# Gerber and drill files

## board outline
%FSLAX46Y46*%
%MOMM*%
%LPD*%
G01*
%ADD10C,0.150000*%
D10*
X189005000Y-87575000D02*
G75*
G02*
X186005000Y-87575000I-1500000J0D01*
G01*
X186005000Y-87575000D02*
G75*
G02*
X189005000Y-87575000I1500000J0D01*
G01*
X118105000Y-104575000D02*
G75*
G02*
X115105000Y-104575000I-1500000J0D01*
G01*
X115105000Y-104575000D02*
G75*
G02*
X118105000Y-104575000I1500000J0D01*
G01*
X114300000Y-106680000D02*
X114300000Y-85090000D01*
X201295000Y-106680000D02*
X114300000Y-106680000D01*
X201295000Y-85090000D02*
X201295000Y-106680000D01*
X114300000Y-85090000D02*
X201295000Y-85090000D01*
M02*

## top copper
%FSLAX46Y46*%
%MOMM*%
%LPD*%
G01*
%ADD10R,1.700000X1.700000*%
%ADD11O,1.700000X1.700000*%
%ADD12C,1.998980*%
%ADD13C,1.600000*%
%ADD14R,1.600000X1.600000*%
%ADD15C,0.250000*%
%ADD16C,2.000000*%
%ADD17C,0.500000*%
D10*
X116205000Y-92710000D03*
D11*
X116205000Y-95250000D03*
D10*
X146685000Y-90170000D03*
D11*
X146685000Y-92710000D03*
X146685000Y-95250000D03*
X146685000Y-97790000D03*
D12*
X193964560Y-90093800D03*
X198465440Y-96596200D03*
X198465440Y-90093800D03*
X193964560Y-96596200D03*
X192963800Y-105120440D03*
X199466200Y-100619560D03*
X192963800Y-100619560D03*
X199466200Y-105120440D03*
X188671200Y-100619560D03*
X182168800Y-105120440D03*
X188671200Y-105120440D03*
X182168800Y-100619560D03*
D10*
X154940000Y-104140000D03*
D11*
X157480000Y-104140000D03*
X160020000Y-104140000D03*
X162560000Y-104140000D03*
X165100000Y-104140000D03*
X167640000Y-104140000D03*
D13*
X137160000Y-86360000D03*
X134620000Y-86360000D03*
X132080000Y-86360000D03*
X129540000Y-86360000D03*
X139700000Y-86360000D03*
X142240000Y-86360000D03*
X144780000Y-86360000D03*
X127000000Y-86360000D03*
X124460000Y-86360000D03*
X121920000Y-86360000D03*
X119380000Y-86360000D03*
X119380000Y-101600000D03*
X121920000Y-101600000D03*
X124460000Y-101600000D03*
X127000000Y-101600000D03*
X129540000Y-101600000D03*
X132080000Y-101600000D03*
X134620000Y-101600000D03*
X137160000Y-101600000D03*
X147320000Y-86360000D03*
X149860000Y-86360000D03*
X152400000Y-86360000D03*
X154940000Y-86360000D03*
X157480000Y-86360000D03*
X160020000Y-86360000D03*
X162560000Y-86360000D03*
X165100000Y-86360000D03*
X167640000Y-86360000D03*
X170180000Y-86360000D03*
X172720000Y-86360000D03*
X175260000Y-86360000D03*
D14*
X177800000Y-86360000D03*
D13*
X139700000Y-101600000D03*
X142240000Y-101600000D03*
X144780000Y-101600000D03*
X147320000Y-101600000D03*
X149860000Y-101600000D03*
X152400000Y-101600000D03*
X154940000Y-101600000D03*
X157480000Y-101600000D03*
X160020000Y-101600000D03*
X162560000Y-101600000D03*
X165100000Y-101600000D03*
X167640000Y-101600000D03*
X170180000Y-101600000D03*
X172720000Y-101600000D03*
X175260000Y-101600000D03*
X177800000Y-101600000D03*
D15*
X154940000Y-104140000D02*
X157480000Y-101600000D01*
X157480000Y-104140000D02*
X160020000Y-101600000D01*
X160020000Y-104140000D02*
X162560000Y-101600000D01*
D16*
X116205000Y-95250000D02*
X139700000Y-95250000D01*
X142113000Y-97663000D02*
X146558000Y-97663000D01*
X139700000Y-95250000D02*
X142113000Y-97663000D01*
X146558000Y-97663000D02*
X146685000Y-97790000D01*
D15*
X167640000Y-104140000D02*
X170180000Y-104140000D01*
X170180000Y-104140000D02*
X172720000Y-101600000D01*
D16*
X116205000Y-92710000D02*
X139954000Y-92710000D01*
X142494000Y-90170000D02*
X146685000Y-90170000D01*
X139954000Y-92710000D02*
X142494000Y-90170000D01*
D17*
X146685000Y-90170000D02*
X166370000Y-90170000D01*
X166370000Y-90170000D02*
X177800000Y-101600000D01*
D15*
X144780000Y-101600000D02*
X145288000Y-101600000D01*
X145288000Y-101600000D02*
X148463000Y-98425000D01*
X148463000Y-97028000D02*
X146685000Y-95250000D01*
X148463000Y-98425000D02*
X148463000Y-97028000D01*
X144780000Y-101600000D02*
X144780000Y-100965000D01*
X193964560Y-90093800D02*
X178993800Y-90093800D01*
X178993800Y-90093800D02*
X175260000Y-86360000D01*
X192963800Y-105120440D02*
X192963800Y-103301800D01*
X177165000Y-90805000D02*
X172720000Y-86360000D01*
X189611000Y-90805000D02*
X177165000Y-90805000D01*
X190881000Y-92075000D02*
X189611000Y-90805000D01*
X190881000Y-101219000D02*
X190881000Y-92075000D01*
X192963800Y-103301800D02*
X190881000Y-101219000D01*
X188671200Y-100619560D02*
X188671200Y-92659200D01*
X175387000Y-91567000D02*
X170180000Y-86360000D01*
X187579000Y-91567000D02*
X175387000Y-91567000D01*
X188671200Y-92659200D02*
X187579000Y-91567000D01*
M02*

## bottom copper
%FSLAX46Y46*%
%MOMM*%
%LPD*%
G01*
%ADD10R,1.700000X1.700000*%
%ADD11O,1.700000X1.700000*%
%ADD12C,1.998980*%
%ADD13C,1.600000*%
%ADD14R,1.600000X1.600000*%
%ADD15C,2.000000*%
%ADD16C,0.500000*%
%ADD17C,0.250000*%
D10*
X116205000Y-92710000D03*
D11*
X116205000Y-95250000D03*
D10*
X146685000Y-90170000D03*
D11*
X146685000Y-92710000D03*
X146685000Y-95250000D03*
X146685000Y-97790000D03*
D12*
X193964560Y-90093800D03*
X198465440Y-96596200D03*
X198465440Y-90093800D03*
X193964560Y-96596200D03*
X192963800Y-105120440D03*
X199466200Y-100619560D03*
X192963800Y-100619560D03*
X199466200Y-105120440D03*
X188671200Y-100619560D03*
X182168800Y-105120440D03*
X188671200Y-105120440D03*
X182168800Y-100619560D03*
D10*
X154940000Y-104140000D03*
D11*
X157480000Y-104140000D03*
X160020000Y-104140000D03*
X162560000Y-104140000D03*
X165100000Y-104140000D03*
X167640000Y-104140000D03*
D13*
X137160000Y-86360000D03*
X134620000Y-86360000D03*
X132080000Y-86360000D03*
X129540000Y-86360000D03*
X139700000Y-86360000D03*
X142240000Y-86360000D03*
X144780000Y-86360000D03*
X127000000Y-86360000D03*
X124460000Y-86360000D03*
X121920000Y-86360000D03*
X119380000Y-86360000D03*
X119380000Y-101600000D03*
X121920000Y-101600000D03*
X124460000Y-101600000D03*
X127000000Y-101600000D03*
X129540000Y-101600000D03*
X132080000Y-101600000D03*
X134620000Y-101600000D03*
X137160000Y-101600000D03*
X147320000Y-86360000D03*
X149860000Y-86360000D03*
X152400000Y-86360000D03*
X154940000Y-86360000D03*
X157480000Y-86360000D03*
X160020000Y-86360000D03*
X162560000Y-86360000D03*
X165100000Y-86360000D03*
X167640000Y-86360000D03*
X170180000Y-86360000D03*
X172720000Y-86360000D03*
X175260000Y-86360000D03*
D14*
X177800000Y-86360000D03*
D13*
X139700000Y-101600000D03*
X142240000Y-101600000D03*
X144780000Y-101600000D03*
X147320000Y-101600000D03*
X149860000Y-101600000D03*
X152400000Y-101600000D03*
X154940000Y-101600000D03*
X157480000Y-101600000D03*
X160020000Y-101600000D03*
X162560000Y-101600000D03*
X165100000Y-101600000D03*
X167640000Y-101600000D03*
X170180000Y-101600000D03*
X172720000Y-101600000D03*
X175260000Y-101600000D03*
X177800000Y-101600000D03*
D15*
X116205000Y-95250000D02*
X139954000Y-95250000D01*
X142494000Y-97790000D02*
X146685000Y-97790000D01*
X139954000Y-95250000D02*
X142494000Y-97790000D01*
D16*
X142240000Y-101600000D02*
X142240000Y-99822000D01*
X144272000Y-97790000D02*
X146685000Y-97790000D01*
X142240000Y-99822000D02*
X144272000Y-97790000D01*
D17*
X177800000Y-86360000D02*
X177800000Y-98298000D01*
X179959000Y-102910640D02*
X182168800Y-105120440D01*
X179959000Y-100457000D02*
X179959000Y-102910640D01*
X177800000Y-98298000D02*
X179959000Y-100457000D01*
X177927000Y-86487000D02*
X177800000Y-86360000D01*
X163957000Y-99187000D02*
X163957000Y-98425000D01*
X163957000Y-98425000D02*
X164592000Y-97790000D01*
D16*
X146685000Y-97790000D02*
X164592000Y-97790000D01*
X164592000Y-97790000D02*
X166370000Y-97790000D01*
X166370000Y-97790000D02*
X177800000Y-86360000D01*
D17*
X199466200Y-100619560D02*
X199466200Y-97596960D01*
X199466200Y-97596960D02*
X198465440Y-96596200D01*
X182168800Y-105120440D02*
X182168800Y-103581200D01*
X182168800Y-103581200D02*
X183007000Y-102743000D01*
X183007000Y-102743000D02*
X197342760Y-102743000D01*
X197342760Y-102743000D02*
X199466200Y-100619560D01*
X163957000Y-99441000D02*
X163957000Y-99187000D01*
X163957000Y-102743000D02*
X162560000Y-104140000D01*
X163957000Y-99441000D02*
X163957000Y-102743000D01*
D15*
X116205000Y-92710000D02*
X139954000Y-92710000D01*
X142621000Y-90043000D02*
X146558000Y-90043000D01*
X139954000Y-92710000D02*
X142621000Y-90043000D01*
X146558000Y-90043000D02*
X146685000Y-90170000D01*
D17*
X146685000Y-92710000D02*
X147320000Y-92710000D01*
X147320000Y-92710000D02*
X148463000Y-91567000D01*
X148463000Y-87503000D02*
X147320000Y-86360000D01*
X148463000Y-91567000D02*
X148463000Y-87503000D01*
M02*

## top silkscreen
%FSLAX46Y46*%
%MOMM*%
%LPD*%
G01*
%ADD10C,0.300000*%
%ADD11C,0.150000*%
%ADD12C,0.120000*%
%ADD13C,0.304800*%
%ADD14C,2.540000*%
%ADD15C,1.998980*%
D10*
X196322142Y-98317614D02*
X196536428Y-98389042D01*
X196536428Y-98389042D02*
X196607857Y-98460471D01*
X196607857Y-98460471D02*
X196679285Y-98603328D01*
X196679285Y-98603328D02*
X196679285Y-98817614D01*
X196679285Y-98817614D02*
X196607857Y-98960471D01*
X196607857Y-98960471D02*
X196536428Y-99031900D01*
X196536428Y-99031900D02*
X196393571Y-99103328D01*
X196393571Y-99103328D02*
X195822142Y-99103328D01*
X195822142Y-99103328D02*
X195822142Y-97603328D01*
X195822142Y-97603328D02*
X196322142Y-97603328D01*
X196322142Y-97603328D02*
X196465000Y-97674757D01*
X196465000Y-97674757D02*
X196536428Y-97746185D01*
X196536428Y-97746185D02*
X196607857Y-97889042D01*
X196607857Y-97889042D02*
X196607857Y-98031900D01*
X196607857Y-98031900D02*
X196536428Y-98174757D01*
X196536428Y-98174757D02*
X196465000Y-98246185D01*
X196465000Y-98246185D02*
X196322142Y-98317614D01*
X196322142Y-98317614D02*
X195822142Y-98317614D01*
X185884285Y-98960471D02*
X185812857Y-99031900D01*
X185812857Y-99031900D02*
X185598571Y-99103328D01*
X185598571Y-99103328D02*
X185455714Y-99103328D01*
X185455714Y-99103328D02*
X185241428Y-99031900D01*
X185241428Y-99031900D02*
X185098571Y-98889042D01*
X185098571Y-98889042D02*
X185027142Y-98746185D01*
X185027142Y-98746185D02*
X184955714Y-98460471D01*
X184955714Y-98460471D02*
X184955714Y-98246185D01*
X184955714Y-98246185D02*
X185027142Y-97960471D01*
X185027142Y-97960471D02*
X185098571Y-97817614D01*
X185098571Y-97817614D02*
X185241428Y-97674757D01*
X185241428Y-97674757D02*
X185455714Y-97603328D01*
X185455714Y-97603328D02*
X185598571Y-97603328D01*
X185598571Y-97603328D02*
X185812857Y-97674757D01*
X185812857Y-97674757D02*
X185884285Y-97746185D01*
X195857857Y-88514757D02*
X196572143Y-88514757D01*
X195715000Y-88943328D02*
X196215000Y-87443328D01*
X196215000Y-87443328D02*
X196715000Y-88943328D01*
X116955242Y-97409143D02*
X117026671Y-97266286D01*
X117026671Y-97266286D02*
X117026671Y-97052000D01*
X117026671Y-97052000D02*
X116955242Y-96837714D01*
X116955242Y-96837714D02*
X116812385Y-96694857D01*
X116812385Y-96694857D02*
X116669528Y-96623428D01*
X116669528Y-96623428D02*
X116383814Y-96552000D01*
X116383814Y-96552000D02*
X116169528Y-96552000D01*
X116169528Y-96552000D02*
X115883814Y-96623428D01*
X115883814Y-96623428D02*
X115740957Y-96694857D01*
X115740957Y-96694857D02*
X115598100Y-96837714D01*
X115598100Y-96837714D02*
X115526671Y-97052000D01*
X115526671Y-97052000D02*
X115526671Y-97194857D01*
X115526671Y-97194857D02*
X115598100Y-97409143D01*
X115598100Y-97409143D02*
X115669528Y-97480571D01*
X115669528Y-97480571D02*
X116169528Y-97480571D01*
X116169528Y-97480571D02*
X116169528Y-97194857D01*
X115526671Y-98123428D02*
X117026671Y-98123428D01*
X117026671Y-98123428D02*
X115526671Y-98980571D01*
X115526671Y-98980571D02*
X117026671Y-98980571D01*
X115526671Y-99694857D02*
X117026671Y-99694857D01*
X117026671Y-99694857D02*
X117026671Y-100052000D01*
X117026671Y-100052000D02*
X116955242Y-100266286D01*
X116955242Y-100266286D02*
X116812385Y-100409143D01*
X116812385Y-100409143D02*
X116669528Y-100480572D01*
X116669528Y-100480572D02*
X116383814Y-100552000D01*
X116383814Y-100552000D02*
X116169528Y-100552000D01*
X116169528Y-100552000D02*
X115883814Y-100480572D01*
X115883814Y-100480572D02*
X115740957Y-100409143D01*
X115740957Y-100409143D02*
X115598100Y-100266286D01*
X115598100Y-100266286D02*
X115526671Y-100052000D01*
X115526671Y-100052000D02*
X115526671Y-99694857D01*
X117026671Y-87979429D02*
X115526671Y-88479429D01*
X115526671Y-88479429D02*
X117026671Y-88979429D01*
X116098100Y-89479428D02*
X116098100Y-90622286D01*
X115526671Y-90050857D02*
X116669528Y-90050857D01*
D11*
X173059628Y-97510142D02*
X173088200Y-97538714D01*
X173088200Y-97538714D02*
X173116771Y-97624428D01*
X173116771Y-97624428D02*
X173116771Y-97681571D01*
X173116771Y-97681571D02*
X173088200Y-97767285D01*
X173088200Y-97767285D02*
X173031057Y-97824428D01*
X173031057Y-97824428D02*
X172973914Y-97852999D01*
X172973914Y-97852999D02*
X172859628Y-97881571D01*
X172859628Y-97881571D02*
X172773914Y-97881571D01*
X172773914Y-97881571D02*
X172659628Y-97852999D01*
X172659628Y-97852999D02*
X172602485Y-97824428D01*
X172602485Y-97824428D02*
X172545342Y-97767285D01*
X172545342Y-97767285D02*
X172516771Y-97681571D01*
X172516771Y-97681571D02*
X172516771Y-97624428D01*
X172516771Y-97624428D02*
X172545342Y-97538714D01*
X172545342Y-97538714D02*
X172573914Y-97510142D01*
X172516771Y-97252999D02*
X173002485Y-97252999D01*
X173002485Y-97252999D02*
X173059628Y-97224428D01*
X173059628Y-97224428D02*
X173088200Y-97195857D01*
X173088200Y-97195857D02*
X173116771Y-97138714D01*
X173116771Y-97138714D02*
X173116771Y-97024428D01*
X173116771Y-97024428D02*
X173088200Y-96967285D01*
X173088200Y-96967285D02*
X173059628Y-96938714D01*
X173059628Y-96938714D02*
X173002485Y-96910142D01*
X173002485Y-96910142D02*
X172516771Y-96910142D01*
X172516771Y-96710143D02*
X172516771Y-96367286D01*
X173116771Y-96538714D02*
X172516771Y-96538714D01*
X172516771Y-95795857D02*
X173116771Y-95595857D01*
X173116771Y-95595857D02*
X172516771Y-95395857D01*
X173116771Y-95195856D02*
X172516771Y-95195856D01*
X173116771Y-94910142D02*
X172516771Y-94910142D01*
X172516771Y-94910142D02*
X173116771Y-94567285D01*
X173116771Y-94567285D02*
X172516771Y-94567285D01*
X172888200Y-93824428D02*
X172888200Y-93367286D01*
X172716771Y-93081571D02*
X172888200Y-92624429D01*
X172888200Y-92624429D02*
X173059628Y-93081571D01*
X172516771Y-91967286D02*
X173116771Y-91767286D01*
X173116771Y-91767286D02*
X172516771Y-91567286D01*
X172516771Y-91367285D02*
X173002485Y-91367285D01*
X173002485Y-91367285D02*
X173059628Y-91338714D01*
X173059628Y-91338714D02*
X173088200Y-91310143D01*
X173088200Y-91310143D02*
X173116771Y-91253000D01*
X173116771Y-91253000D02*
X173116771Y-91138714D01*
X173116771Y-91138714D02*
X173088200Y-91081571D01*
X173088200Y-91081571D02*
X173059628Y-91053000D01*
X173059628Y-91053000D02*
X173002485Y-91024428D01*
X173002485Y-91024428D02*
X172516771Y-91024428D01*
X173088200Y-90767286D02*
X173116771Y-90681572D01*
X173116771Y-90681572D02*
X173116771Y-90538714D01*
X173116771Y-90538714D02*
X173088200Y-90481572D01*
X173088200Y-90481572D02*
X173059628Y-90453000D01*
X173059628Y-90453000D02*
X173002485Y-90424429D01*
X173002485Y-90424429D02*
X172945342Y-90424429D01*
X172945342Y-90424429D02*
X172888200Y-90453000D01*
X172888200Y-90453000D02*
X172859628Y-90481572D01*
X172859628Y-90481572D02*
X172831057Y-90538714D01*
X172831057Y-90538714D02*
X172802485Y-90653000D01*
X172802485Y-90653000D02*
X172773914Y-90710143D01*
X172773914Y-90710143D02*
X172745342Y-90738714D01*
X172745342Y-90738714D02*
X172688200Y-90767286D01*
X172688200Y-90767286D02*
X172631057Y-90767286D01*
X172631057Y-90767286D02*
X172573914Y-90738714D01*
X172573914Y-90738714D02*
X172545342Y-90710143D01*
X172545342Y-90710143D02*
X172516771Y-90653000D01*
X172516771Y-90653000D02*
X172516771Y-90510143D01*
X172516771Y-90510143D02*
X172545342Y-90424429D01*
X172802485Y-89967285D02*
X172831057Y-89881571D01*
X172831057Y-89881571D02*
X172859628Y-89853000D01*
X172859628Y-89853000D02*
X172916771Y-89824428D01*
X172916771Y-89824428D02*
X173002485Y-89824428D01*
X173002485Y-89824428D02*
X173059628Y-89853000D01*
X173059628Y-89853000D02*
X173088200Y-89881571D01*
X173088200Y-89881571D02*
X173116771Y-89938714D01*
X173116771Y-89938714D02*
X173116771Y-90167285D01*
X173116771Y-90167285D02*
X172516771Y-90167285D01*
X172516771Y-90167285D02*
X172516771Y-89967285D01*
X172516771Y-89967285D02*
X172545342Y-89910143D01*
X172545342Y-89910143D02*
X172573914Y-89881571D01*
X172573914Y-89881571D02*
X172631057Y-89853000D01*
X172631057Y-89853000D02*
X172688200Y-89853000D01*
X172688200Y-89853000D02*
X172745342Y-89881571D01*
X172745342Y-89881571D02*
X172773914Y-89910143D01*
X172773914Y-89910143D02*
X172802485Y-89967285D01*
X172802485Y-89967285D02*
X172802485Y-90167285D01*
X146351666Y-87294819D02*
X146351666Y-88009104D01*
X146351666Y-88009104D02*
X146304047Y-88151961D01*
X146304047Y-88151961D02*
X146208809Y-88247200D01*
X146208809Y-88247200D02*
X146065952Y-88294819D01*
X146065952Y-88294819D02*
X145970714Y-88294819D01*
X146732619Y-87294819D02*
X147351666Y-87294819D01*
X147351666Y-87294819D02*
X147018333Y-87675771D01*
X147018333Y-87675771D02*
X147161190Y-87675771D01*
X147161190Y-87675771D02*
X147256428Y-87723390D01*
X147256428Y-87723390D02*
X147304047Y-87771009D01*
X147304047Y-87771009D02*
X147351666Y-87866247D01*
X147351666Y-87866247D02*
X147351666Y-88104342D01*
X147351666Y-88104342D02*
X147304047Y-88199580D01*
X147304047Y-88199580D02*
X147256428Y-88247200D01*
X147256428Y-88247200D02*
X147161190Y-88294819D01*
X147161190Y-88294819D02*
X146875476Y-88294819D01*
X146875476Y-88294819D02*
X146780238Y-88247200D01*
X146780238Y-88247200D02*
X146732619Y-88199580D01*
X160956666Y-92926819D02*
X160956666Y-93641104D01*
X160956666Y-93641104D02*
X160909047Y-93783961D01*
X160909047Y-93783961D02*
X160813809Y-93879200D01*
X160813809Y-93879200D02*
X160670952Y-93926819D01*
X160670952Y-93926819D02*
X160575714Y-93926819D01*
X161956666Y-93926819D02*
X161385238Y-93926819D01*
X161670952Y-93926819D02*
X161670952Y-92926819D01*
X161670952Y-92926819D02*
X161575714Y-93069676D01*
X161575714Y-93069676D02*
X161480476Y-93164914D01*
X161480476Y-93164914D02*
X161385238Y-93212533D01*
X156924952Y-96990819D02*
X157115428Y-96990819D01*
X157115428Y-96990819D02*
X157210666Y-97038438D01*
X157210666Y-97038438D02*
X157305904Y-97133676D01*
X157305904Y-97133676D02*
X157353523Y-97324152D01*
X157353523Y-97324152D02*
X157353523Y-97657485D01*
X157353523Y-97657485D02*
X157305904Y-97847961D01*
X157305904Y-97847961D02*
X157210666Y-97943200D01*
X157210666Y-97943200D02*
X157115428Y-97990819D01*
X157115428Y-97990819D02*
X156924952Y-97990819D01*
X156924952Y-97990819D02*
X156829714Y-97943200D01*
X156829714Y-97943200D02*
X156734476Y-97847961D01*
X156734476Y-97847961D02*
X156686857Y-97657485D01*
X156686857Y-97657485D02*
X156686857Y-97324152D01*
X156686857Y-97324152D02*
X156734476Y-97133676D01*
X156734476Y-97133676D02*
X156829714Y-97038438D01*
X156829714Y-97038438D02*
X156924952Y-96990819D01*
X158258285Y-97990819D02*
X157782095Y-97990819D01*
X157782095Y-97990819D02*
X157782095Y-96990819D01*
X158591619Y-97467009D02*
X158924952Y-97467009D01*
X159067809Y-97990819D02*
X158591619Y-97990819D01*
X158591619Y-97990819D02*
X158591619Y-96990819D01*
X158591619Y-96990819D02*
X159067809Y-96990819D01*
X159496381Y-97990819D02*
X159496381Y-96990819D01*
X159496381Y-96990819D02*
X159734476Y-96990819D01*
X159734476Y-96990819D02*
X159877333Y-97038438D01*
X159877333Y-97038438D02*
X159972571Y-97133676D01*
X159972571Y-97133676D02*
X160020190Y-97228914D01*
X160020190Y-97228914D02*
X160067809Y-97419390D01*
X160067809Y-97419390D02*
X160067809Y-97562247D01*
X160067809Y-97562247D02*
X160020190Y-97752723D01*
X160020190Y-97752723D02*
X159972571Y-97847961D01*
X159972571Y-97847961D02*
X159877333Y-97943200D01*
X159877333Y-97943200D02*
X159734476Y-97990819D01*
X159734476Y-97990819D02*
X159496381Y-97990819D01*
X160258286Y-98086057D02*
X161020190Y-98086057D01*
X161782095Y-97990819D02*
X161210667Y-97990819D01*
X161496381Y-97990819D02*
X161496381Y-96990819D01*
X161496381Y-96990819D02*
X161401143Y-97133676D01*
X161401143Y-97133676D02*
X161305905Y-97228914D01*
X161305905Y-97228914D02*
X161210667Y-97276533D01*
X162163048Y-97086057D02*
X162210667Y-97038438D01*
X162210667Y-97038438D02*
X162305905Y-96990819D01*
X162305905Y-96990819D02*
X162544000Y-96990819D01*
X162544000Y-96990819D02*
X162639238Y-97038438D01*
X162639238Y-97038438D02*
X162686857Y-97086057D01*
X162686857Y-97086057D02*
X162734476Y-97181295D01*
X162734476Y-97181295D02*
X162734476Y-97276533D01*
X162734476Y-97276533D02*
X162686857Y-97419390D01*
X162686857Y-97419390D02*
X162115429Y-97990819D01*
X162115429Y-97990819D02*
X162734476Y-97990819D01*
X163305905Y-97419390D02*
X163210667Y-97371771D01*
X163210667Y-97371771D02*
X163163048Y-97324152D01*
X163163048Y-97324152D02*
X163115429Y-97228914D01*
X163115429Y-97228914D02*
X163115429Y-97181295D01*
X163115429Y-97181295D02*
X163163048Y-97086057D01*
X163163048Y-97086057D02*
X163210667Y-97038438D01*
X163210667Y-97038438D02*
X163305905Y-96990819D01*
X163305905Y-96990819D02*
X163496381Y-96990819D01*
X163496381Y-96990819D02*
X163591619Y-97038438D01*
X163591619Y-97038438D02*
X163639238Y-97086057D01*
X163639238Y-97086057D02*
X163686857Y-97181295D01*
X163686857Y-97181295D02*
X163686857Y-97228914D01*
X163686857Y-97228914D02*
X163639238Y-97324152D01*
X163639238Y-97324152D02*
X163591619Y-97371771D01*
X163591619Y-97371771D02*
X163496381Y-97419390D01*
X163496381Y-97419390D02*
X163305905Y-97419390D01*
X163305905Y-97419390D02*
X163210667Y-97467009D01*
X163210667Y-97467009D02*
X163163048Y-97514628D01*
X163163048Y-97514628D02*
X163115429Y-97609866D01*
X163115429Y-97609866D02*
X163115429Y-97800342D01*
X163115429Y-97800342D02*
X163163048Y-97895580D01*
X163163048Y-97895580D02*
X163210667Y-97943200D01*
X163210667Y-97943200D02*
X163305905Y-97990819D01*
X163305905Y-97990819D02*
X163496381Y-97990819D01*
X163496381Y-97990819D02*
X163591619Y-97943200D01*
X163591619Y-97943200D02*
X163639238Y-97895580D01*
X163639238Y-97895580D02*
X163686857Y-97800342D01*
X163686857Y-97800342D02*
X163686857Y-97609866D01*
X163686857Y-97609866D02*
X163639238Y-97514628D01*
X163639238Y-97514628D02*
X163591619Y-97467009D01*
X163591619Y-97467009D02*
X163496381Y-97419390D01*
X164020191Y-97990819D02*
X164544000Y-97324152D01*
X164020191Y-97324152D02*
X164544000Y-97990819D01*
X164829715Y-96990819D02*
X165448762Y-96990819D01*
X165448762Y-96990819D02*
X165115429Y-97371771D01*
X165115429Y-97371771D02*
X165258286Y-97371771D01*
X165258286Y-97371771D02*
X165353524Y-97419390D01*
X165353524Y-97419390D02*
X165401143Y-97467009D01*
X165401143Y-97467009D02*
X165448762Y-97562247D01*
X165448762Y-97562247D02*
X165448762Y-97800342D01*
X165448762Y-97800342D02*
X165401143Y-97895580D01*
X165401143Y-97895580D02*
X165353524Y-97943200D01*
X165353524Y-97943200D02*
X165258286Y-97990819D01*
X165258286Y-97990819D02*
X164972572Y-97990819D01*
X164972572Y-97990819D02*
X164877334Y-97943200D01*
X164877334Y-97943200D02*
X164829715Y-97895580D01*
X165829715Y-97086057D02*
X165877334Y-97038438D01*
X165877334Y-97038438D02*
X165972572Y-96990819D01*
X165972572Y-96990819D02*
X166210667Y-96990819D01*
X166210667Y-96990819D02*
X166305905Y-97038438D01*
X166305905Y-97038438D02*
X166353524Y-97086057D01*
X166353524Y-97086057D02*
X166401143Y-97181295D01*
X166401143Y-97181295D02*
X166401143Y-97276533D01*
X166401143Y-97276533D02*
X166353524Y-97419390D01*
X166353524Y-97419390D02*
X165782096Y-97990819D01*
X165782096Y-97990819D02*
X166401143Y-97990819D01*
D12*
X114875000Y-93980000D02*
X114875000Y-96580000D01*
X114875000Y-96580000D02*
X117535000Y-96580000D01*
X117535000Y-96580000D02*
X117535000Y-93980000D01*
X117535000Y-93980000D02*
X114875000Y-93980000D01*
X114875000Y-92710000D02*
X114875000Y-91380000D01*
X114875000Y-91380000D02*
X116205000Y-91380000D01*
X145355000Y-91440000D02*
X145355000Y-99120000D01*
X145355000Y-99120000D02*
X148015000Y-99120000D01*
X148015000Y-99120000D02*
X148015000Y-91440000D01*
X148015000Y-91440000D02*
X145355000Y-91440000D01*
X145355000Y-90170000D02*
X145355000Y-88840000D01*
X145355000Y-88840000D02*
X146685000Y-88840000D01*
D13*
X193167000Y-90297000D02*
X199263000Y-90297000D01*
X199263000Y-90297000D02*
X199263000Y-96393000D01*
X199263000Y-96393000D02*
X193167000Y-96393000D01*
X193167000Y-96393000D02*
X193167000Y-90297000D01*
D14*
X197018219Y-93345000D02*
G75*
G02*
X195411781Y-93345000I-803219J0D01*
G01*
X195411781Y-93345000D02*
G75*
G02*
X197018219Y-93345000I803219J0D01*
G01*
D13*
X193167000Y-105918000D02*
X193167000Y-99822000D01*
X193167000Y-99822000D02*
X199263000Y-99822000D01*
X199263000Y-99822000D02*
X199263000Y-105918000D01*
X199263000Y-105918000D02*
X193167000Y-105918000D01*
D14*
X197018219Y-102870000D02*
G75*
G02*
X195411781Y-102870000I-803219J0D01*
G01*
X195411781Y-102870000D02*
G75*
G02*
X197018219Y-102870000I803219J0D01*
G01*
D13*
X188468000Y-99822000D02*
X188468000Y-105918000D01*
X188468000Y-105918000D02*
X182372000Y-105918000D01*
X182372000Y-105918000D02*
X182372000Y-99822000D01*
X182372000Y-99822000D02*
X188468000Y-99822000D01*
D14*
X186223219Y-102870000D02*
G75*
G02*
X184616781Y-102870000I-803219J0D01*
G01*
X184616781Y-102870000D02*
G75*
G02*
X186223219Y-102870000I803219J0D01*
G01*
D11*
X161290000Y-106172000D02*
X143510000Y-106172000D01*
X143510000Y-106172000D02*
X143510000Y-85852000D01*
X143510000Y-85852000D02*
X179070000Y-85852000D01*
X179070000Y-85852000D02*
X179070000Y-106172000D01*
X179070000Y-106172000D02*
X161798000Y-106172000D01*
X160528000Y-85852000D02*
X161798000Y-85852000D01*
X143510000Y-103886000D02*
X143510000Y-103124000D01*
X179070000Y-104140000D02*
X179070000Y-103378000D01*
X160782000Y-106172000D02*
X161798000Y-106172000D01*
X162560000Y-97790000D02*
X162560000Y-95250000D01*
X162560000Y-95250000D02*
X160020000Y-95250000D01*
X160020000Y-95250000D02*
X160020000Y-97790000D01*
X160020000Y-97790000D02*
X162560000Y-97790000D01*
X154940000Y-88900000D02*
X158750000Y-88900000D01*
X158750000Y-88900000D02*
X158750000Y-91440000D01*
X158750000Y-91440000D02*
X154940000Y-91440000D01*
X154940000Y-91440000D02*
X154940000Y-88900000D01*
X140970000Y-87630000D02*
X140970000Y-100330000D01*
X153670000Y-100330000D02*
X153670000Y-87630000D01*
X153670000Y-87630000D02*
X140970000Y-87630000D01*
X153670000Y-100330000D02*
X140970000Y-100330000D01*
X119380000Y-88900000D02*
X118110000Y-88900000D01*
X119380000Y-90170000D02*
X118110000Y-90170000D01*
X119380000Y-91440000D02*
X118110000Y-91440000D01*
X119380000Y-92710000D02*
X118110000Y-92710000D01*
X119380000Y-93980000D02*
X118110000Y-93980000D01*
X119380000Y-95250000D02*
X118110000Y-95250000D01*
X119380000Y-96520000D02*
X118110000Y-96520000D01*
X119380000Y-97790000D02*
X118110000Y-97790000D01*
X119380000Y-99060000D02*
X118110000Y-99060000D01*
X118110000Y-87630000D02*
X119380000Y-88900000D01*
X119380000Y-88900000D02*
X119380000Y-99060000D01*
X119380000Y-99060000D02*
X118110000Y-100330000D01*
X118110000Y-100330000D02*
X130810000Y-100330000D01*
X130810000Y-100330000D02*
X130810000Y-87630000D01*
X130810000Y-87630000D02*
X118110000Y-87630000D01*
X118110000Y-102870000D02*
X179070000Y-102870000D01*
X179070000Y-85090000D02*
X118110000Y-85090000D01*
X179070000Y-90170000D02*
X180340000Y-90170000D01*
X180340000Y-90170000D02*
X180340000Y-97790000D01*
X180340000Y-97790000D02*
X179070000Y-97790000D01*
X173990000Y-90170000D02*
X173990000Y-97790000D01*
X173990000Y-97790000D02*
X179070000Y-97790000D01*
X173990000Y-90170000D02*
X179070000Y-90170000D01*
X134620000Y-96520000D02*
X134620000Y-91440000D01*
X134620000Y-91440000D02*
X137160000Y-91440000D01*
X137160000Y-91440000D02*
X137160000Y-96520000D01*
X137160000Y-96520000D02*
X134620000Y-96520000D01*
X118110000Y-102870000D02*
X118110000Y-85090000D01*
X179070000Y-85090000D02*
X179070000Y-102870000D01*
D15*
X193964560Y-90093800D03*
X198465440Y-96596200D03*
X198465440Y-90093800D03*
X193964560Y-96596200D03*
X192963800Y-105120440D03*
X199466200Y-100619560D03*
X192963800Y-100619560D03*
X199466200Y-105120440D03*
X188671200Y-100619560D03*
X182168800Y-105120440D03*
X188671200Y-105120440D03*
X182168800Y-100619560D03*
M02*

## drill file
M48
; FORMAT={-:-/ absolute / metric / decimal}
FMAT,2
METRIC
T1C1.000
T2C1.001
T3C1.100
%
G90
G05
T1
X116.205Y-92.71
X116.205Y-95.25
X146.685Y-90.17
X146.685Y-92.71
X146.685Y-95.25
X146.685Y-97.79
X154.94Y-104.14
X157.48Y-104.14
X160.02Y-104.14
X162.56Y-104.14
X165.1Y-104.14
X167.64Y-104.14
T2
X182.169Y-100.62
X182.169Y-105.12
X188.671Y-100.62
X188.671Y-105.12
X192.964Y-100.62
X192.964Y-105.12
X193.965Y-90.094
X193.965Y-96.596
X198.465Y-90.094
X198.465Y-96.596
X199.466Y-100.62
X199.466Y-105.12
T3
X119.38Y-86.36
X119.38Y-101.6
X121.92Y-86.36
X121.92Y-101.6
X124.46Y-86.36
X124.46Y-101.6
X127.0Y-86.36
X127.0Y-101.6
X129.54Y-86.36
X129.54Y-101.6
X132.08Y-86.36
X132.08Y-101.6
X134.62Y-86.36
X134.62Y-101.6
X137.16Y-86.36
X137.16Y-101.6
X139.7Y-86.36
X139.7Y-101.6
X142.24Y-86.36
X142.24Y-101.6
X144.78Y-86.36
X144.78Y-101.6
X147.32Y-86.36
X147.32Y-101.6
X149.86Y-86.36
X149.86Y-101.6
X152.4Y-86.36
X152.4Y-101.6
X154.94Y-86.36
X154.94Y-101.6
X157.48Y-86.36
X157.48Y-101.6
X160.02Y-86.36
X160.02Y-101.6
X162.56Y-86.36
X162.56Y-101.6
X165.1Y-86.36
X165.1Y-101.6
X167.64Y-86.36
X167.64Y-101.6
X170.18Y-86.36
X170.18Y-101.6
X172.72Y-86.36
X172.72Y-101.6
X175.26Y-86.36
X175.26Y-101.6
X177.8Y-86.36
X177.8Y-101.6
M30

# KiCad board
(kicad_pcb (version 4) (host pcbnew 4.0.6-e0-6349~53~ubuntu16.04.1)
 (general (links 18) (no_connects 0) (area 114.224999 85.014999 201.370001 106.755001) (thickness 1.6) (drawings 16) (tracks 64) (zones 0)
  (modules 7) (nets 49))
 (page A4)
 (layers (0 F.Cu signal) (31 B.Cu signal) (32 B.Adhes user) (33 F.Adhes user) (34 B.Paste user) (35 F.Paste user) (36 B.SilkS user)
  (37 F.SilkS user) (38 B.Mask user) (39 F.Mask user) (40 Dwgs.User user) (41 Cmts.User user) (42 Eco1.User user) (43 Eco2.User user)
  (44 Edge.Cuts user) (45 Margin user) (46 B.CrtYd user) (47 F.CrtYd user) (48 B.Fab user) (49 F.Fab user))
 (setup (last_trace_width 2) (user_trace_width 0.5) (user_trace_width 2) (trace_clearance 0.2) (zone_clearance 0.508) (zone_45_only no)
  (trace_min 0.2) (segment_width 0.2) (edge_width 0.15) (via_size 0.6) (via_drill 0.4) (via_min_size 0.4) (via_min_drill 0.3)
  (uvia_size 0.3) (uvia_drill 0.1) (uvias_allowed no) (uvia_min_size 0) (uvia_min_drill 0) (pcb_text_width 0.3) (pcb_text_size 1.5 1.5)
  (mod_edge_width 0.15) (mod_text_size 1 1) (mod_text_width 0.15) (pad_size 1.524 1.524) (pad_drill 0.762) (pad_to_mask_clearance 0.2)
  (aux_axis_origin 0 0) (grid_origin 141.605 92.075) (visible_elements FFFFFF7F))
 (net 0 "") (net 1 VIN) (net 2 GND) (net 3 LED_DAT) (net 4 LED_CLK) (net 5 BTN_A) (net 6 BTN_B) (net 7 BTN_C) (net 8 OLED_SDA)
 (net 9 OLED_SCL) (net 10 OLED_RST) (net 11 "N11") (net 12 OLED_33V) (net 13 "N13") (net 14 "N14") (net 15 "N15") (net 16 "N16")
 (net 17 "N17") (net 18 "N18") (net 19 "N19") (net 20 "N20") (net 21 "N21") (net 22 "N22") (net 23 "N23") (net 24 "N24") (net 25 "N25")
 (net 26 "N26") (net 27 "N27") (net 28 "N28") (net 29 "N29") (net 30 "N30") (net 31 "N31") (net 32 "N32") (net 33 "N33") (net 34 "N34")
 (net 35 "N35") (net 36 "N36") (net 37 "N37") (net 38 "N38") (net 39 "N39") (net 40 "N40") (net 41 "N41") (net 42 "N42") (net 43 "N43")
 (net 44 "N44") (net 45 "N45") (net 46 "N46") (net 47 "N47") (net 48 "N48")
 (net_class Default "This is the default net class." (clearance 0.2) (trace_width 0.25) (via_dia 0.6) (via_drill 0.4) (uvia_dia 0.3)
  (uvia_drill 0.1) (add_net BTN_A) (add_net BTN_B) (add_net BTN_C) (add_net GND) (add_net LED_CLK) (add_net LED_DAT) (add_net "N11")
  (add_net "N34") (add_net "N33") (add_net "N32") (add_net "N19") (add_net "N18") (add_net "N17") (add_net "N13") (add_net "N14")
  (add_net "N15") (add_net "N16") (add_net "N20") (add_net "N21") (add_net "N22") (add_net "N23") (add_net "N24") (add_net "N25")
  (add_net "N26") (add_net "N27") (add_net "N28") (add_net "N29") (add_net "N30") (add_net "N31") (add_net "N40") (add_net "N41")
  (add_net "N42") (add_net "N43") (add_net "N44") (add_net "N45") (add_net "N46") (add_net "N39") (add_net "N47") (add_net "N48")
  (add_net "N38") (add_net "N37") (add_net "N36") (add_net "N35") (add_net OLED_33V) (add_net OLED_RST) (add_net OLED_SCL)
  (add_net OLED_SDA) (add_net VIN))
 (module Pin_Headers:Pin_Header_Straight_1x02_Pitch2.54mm (layer F.Cu) (at 116.205 92.71)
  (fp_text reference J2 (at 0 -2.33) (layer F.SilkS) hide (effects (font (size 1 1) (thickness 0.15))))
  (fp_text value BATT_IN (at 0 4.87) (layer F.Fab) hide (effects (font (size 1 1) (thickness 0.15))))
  (fp_line (start -1.33 1.27) (end -1.33 3.87) (layer F.SilkS) (width 0.12))
  (fp_line (start -1.33 3.87) (end 1.33 3.87) (layer F.SilkS) (width 0.12))
  (fp_line (start 1.33 3.87) (end 1.33 1.27) (layer F.SilkS) (width 0.12))
  (fp_line (start 1.33 1.27) (end -1.33 1.27) (layer F.SilkS) (width 0.12))
  (fp_line (start -1.33 0) (end -1.33 -1.33) (layer F.SilkS) (width 0.12))
  (fp_line (start -1.33 -1.33) (end 0 -1.33) (layer F.SilkS) (width 0.12))
  (pad 1 thru_hole rect (at 0 0) (size 1.7 1.7) (drill 1) (layers *.Cu *.Mask) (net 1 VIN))
  (pad 2 thru_hole oval (at 0 2.54) (size 1.7 1.7) (drill 1) (layers *.Cu *.Mask) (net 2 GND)))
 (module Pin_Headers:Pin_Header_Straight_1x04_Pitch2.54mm (layer F.Cu) (at 146.685 90.17)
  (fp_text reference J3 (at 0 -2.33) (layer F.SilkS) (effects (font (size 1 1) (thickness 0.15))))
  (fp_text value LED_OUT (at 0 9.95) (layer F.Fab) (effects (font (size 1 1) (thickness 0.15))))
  (fp_line (start -1.33 1.27) (end -1.33 8.95) (layer F.SilkS) (width 0.12))
  (fp_line (start -1.33 8.95) (end 1.33 8.95) (layer F.SilkS) (width 0.12))
  (fp_line (start 1.33 8.95) (end 1.33 1.27) (layer F.SilkS) (width 0.12))
  (fp_line (start 1.33 1.27) (end -1.33 1.27) (layer F.SilkS) (width 0.12))
  (fp_line (start -1.33 0) (end -1.33 -1.33) (layer F.SilkS) (width 0.12))
  (fp_line (start -1.33 -1.33) (end 0 -1.33) (layer F.SilkS) (width 0.12))
  (pad 1 thru_hole rect (at 0 0) (size 1.7 1.7) (drill 1) (layers *.Cu *.Mask) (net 1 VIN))
  (pad 2 thru_hole oval (at 0 2.54) (size 1.7 1.7) (drill 1) (layers *.Cu *.Mask) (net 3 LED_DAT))
  (pad 3 thru_hole oval (at 0 5.08) (size 1.7 1.7) (drill 1) (layers *.Cu *.Mask) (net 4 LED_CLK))
  (pad 4 thru_hole oval (at 0 7.62) (size 1.7 1.7) (drill 1) (layers *.Cu *.Mask) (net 2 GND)))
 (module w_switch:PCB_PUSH (layer F.Cu) (at 196.215 93.345)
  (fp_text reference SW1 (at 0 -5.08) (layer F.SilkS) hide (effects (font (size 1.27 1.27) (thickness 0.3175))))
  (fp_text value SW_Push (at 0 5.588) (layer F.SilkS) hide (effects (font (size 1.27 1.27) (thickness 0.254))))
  (fp_line (start -3.048 -3.048) (end 3.048 -3.048) (layer F.SilkS) (width 0.3048))
  (fp_line (start 3.048 -3.048) (end 3.048 3.048) (layer F.SilkS) (width 0.3048))
  (fp_line (start 3.048 3.048) (end -3.048 3.048) (layer F.SilkS) (width 0.3048))
  (fp_line (start -3.048 3.048) (end -3.048 -3.048) (layer F.SilkS) (width 0.3048))
  (fp_circle (center 0 0) (end -0.762 0.254) (layer F.SilkS) (width 2.54))
  (pad 1 thru_hole circle (at -2.25044 -3.2512) (size 1.99898 1.99898) (drill 1.00076) (layers *.Cu *.Mask F.SilkS) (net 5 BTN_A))
  (pad 2 thru_hole circle (at 2.25044 3.2512) (size 1.99898 1.99898) (drill 1.00076) (layers *.Cu *.Mask F.SilkS) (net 2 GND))
  (pad 4 thru_hole circle (at 2.25044 -3.2512) (size 1.99898 1.99898) (drill 1.00076) (layers *.Cu *.Mask F.SilkS))
  (pad 3 thru_hole circle (at -2.25044 3.2512) (size 1.99898 1.99898) (drill 1.00076) (layers *.Cu *.Mask F.SilkS)))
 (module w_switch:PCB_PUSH (layer F.Cu) (at 196.215 102.87 90)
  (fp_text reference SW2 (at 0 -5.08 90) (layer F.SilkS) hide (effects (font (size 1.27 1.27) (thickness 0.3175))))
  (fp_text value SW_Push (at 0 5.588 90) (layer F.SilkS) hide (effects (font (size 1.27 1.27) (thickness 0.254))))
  (fp_line (start -3.048 -3.048) (end 3.048 -3.048) (layer F.SilkS) (width 0.3048))
  (fp_line (start 3.048 -3.048) (end 3.048 3.048) (layer F.SilkS) (width 0.3048))
  (fp_line (start 3.048 3.048) (end -3.048 3.048) (layer F.SilkS) (width 0.3048))
  (fp_line (start -3.048 3.048) (end -3.048 -3.048) (layer F.SilkS) (width 0.3048))
  (fp_circle (center 0 0) (end -0.762 0.254) (layer F.SilkS) (width 2.54))
  (pad 1 thru_hole circle (at -2.25044 -3.2512 90) (size 1.99898 1.99898) (drill 1.00076) (layers *.Cu *.Mask F.SilkS) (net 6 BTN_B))
  (pad 2 thru_hole circle (at 2.25044 3.2512 90) (size 1.99898 1.99898) (drill 1.00076) (layers *.Cu *.Mask F.SilkS) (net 2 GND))
  (pad 4 thru_hole circle (at 2.25044 -3.2512 90) (size 1.99898 1.99898) (drill 1.00076) (layers *.Cu *.Mask F.SilkS))
  (pad 3 thru_hole circle (at -2.25044 3.2512 90) (size 1.99898 1.99898) (drill 1.00076) (layers *.Cu *.Mask F.SilkS)))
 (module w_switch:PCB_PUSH (layer F.Cu) (at 185.42 102.87 270)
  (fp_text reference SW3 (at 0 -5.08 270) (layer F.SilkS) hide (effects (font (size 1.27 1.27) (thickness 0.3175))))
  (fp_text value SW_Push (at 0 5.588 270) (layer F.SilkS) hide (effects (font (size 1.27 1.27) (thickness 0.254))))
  (fp_line (start -3.048 -3.048) (end 3.048 -3.048) (layer F.SilkS) (width 0.3048))
  (fp_line (start 3.048 -3.048) (end 3.048 3.048) (layer F.SilkS) (width 0.3048))
  (fp_line (start 3.048 3.048) (end -3.048 3.048) (layer F.SilkS) (width 0.3048))
  (fp_line (start -3.048 3.048) (end -3.048 -3.048) (layer F.SilkS) (width 0.3048))
  (fp_circle (center 0 0) (end -0.762 0.254) (layer F.SilkS) (width 2.54))
  (pad 1 thru_hole circle (at -2.25044 -3.2512 270) (size 1.99898 1.99898) (drill 1.00076) (layers *.Cu *.Mask F.SilkS) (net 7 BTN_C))
  (pad 2 thru_hole circle (at 2.25044 3.2512 270) (size 1.99898 1.99898) (drill 1.00076) (layers *.Cu *.Mask F.SilkS) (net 2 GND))
  (pad 4 thru_hole circle (at 2.25044 -3.2512 270) (size 1.99898 1.99898) (drill 1.00076) (layers *.Cu *.Mask F.SilkS))
  (pad 3 thru_hole circle (at -2.25044 3.2512 270) (size 1.99898 1.99898) (drill 1.00076) (layers *.Cu *.Mask F.SilkS)))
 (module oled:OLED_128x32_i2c (layer F.Cu) (at 161.29 104.14)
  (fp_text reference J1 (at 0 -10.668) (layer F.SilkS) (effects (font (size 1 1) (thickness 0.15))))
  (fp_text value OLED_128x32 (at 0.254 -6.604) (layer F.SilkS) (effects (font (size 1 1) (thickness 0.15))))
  (fp_line (start 0 2.032) (end -17.78 2.032) (layer F.SilkS) (width 0.15))
  (fp_line (start -17.78 2.032) (end -17.78 -18.288) (layer F.SilkS) (width 0.15))
  (fp_line (start -17.78 -18.288) (end 17.78 -18.288) (layer F.SilkS) (width 0.15))
  (fp_line (start 17.78 -18.288) (end 17.78 2.032) (layer F.SilkS) (width 0.15))
  (fp_line (start 17.78 2.032) (end 0.508 2.032) (layer F.SilkS) (width 0.15))
  (fp_line (start -0.762 -18.288) (end 0.508 -18.288) (layer F.SilkS) (width 0.15))
  (fp_line (start -17.78 -0.254) (end -17.78 -1.016) (layer F.SilkS) (width 0.15))
  (fp_line (start 17.78 0) (end 17.78 -0.762) (layer F.SilkS) (width 0.15))
  (fp_line (start -0.508 2.032) (end 0.508 2.032) (layer F.SilkS) (width 0.15))
  (pad 1 thru_hole rect (at -6.35 0) (size 1.7 1.7) (drill 1) (layers *.Cu *.Mask) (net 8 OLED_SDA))
  (pad 2 thru_hole oval (at -3.81 0) (size 1.7 1.7) (drill 1) (layers *.Cu *.Mask) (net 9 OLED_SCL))
  (pad 3 thru_hole oval (at -1.27 0) (size 1.7 1.7) (drill 1) (layers *.Cu *.Mask) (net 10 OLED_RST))
  (pad 4 thru_hole oval (at 1.27 0) (size 1.7 1.7) (drill 1) (layers *.Cu *.Mask) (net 2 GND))
  (pad 5 thru_hole oval (at 3.81 0) (size 1.7 1.7) (drill 1) (layers *.Cu *.Mask) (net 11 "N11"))
  (pad 6 thru_hole oval (at 6.35 0) (size 1.7 1.7) (drill 1) (layers *.Cu *.Mask) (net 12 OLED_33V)))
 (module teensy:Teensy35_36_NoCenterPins (layer F.Cu) (at 148.59 93.98 180)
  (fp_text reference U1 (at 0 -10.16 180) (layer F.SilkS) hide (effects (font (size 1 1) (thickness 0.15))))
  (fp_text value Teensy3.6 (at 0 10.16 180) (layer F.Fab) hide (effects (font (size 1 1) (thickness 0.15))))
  (fp_line (start -13.97 -3.81) (end -13.97 -1.27) (layer F.SilkS) (width 0.15))
  (fp_line (start -13.97 -1.27) (end -11.43 -1.27) (layer F.SilkS) (width 0.15))
  (fp_line (start -11.43 -1.27) (end -11.43 -3.81) (layer F.SilkS) (width 0.15))
  (fp_line (start -11.43 -3.81) (end -13.97 -3.81) (layer F.SilkS) (width 0.15))
  (fp_line (start -6.35 5.08) (end -10.16 5.08) (layer F.SilkS) (width 0.15))
  (fp_line (start -10.16 5.08) (end -10.16 2.54) (layer F.SilkS) (width 0.15))
  (fp_line (start -10.16 2.54) (end -6.35 2.54) (layer F.SilkS) (width 0.15))
  (fp_line (start -6.35 2.54) (end -6.35 5.08) (layer F.SilkS) (width 0.15))
  (fp_line (start 7.62 6.35) (end 7.62 -6.35) (layer F.SilkS) (width 0.15))
  (fp_line (start -5.08 -6.35) (end -5.08 6.35) (layer F.SilkS) (width 0.15))
  (fp_line (start -5.08 6.35) (end 7.62 6.35) (layer F.SilkS) (width 0.15))
  (fp_line (start -5.08 -6.35) (end 7.62 -6.35) (layer F.SilkS) (width 0.15))
  (fp_line (start 29.21 5.08) (end 30.48 5.08) (layer F.SilkS) (width 0.15))
  (fp_line (start 29.21 3.81) (end 30.48 3.81) (layer F.SilkS) (width 0.15))
  (fp_line (start 29.21 2.54) (end 30.48 2.54) (layer F.SilkS) (width 0.15))
  (fp_line (start 29.21 1.27) (end 30.48 1.27) (layer F.SilkS) (width 0.15))
  (fp_line (start 29.21 0) (end 30.48 0) (layer F.SilkS) (width 0.15))
  (fp_line (start 29.21 -1.27) (end 30.48 -1.27) (layer F.SilkS) (width 0.15))
  (fp_line (start 29.21 -2.54) (end 30.48 -2.54) (layer F.SilkS) (width 0.15))
  (fp_line (start 29.21 -3.81) (end 30.48 -3.81) (layer F.SilkS) (width 0.15))
  (fp_line (start 29.21 -5.08) (end 30.48 -5.08) (layer F.SilkS) (width 0.15))
  (fp_line (start 30.48 6.35) (end 29.21 5.08) (layer F.SilkS) (width 0.15))
  (fp_line (start 29.21 5.08) (end 29.21 -5.08) (layer F.SilkS) (width 0.15))
  (fp_line (start 29.21 -5.08) (end 30.48 -6.35) (layer F.SilkS) (width 0.15))
  (fp_line (start 30.48 -6.35) (end 17.78 -6.35) (layer F.SilkS) (width 0.15))
  (fp_line (start 17.78 -6.35) (end 17.78 6.35) (layer F.SilkS) (width 0.15))
  (fp_line (start 17.78 6.35) (end 30.48 6.35) (layer F.SilkS) (width 0.15))
  (fp_line (start 30.48 -8.89) (end -30.48 -8.89) (layer F.SilkS) (width 0.15))
  (fp_line (start -30.48 8.89) (end 30.48 8.89) (layer F.SilkS) (width 0.15))
  (fp_line (start -30.48 3.81) (end -31.75 3.81) (layer F.SilkS) (width 0.15))
  (fp_line (start -31.75 3.81) (end -31.75 -3.81) (layer F.SilkS) (width 0.15))
  (fp_line (start -31.75 -3.81) (end -30.48 -3.81) (layer F.SilkS) (width 0.15))
  (fp_line (start -25.4 3.81) (end -25.4 -3.81) (layer F.SilkS) (width 0.15))
  (fp_line (start -25.4 -3.81) (end -30.48 -3.81) (layer F.SilkS) (width 0.15))
  (fp_line (start -25.4 3.81) (end -30.48 3.81) (layer F.SilkS) (width 0.15))
  (fp_line (start 13.97 -2.54) (end 13.97 2.54) (layer F.SilkS) (width 0.15))
  (fp_line (start 13.97 2.54) (end 11.43 2.54) (layer F.SilkS) (width 0.15))
  (fp_line (start 11.43 2.54) (end 11.43 -2.54) (layer F.SilkS) (width 0.15))
  (fp_line (start 11.43 -2.54) (end 13.97 -2.54) (layer F.SilkS) (width 0.15))
  (fp_line (start 30.48 -8.89) (end 30.48 8.89) (layer F.SilkS) (width 0.15))
  (fp_line (start -30.48 8.89) (end -30.48 -8.89) (layer F.SilkS) (width 0.15))
  (pad 17 thru_hole circle (at 11.43 7.62 180) (size 1.6 1.6) (drill 1.1) (layers *.Cu *.Mask) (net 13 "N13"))
  (pad 18 thru_hole circle (at 13.97 7.62 180) (size 1.6 1.6) (drill 1.1) (layers *.Cu *.Mask) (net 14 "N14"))
  (pad 19 thru_hole circle (at 16.51 7.62 180) (size 1.6 1.6) (drill 1.1) (layers *.Cu *.Mask) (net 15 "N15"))
  (pad 20 thru_hole circle (at 19.05 7.62 180) (size 1.6 1.6) (drill 1.1) (layers *.Cu *.Mask) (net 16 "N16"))
  (pad 16 thru_hole circle (at 8.89 7.62 180) (size 1.6 1.6) (drill 1.1) (layers *.Cu *.Mask) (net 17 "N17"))
  (pad 15 thru_hole circle (at 6.35 7.62 180) (size 1.6 1.6) (drill 1.1) (layers *.Cu *.Mask) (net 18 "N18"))
  (pad 14 thru_hole circle (at 3.81 7.62 180) (size 1.6 1.6) (drill 1.1) (layers *.Cu *.Mask) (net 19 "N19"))
  (pad 21 thru_hole circle (at 21.59 7.62 180) (size 1.6 1.6) (drill 1.1) (layers *.Cu *.Mask) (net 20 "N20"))
  (pad 22 thru_hole circle (at 24.13 7.62 180) (size 1.6 1.6) (drill 1.1) (layers *.Cu *.Mask) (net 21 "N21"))
  (pad 23 thru_hole circle (at 26.67 7.62 180) (size 1.6 1.6) (drill 1.1) (layers *.Cu *.Mask) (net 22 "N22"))
  (pad 24 thru_hole circle (at 29.21 7.62 180) (size 1.6 1.6) (drill 1.1) (layers *.Cu *.Mask) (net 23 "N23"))
  (pad 30 thru_hole circle (at 29.21 -7.62 180) (size 1.6 1.6) (drill 1.1) (layers *.Cu *.Mask) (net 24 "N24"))
  (pad 31 thru_hole circle (at 26.67 -7.62 180) (size 1.6 1.6) (drill 1.1) (layers *.Cu *.Mask) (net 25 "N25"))
  (pad 32 thru_hole circle (at 24.13 -7.62 180) (size 1.6 1.6) (drill 1.1) (layers *.Cu *.Mask) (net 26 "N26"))
  (pad 33 thru_hole circle (at 21.59 -7.62 180) (size 1.6 1.6) (drill 1.1) (layers *.Cu *.Mask) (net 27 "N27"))
  (pad 34 thru_hole circle (at 19.05 -7.62 180) (size 1.6 1.6) (drill 1.1) (layers *.Cu *.Mask) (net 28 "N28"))
  (pad 35 thru_hole circle (at 16.51 -7.62 180) (size 1.6 1.6) (drill 1.1) (layers *.Cu *.Mask) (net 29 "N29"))
  (pad 36 thru_hole circle (at 13.97 -7.62 180) (size 1.6 1.6) (drill 1.1) (layers *.Cu *.Mask) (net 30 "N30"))
  (pad 37 thru_hole circle (at 11.43 -7.62 180) (size 1.6 1.6) (drill 1.1) (layers *.Cu *.Mask) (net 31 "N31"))
  (pad 13 thru_hole circle (at 1.27 7.62 180) (size 1.6 1.6) (drill 1.1) (layers *.Cu *.Mask) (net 3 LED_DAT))
  (pad 12 thru_hole circle (at -1.27 7.62 180) (size 1.6 1.6) (drill 1.1) (layers *.Cu *.Mask) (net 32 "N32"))
  (pad 11 thru_hole circle (at -3.81 7.62 180) (size 1.6 1.6) (drill 1.1) (layers *.Cu *.Mask) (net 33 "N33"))
  (pad 10 thru_hole circle (at -6.35 7.62 180) (size 1.6 1.6) (drill 1.1) (layers *.Cu *.Mask) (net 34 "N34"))
  (pad 9 thru_hole circle (at -8.89 7.62 180) (size 1.6 1.6) (drill 1.1) (layers *.Cu *.Mask) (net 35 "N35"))
  (pad 8 thru_hole circle (at -11.43 7.62 180) (size 1.6 1.6) (drill 1.1) (layers *.Cu *.Mask) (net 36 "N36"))
  (pad 7 thru_hole circle (at -13.97 7.62 180) (size 1.6 1.6) (drill 1.1) (layers *.Cu *.Mask) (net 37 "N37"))
  (pad 6 thru_hole circle (at -16.51 7.62 180) (size 1.6 1.6) (drill 1.1) (layers *.Cu *.Mask) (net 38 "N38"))
  (pad 5 thru_hole circle (at -19.05 7.62 180) (size 1.6 1.6) (drill 1.1) (layers *.Cu *.Mask) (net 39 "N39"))
  (pad 4 thru_hole circle (at -21.59 7.62 180) (size 1.6 1.6) (drill 1.1) (layers *.Cu *.Mask) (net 7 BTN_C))
  (pad 3 thru_hole circle (at -24.13 7.62 180) (size 1.6 1.6) (drill 1.1) (layers *.Cu *.Mask) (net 6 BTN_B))
  (pad 2 thru_hole circle (at -26.67 7.62 180) (size 1.6 1.6) (drill 1.1) (layers *.Cu *.Mask) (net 5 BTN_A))
  (pad 1 thru_hole rect (at -29.21 7.62 180) (size 1.6 1.6) (drill 1.1) (layers *.Cu *.Mask) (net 2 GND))
  (pad 38 thru_hole circle (at 8.89 -7.62 180) (size 1.6 1.6) (drill 1.1) (layers *.Cu *.Mask) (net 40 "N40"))
  (pad 39 thru_hole circle (at 6.35 -7.62 180) (size 1.6 1.6) (drill 1.1) (layers *.Cu *.Mask) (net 2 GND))
  (pad 40 thru_hole circle (at 3.81 -7.62 180) (size 1.6 1.6) (drill 1.1) (layers *.Cu *.Mask) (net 4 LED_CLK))
  (pad 41 thru_hole circle (at 1.27 -7.62 180) (size 1.6 1.6) (drill 1.1) (layers *.Cu *.Mask) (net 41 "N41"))
  (pad 42 thru_hole circle (at -1.27 -7.62 180) (size 1.6 1.6) (drill 1.1) (layers *.Cu *.Mask) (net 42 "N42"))
  (pad 43 thru_hole circle (at -3.81 -7.62 180) (size 1.6 1.6) (drill 1.1) (layers *.Cu *.Mask) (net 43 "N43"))
  (pad 44 thru_hole circle (at -6.35 -7.62 180) (size 1.6 1.6) (drill 1.1) (layers *.Cu *.Mask) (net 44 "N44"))
  (pad 45 thru_hole circle (at -8.89 -7.62 180) (size 1.6 1.6) (drill 1.1) (layers *.Cu *.Mask) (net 8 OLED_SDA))
  (pad 46 thru_hole circle (at -11.43 -7.62 180) (size 1.6 1.6) (drill 1.1) (layers *.Cu *.Mask) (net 9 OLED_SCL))
  (pad 47 thru_hole circle (at -13.97 -7.62 180) (size 1.6 1.6) (drill 1.1) (layers *.Cu *.Mask) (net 10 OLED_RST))
  (pad 48 thru_hole circle (at -16.51 -7.62 180) (size 1.6 1.6) (drill 1.1) (layers *.Cu *.Mask) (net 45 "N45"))
  (pad 49 thru_hole circle (at -19.05 -7.62 180) (size 1.6 1.6) (drill 1.1) (layers *.Cu *.Mask) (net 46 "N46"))
  (pad 50 thru_hole circle (at -21.59 -7.62 180) (size 1.6 1.6) (drill 1.1) (layers *.Cu *.Mask) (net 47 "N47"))
  (pad 51 thru_hole circle (at -24.13 -7.62 180) (size 1.6 1.6) (drill 1.1) (layers *.Cu *.Mask) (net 12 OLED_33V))
  (pad 52 thru_hole circle (at -26.67 -7.62 180) (size 1.6 1.6) (drill 1.1) (layers *.Cu *.Mask) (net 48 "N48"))
  (pad 53 thru_hole circle (at -29.21 -7.62 180) (size 1.6 1.6) (drill 1.1) (layers *.Cu *.Mask) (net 1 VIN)))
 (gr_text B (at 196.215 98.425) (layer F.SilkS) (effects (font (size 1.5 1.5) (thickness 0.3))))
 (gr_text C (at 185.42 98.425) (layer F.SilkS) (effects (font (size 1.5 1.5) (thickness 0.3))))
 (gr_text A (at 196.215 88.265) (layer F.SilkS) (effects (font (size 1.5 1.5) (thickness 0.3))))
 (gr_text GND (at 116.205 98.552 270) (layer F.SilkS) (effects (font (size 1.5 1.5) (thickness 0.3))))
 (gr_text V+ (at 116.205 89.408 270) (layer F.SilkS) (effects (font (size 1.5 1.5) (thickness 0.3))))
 (gr_circle (center 187.505 87.575) (end 189.005 87.575) (layer Edge.Cuts) (width 0.15))
 (gr_circle (center 116.605 104.575) (end 118.105 104.575) (layer Edge.Cuts) (width 0.15))
 (gr_line (start 114.3 106.68) (end 114.3 85.09) (angle 90) (layer Edge.Cuts) (width 0.15))
 (gr_line (start 201.295 106.68) (end 114.3 106.68) (angle 90) (layer Edge.Cuts) (width 0.15))
 (gr_line (start 201.295 85.09) (end 201.295 106.68) (angle 90) (layer Edge.Cuts) (width 0.15))
 (gr_line (start 114.3 85.09) (end 201.295 85.09) (angle 90) (layer Edge.Cuts) (width 0.15))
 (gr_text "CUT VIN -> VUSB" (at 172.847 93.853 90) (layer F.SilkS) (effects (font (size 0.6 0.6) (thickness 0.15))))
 (segment (start 154.94 104.14) (end 157.48 101.6) (width 0.25) (layer F.Cu) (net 8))
 (segment (start 157.48 104.14) (end 160.02 101.6) (width 0.25) (layer F.Cu) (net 9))
 (segment (start 160.02 104.14) (end 162.56 101.6) (width 0.25) (layer F.Cu) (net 10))
 (segment (start 116.205 95.25) (end 139.7 95.25) (width 2) (layer F.Cu) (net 2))
 (segment (start 142.113 97.663) (end 146.558 97.663) (width 2) (layer F.Cu) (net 2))
 (segment (start 139.7 95.25) (end 142.113 97.663) (width 2) (layer F.Cu) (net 2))
 (segment (start 146.558 97.663) (end 146.685 97.79) (width 2) (layer F.Cu) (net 2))
 (segment (start 116.205 95.25) (end 139.954 95.25) (width 2) (layer B.Cu) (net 2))
 (segment (start 142.494 97.79) (end 146.685 97.79) (width 2) (layer B.Cu) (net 2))
 (segment (start 139.954 95.25) (end 142.494 97.79) (width 2) (layer B.Cu) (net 2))
 (segment (start 142.24 101.6) (end 142.24 99.822) (width 0.5) (layer B.Cu) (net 2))
 (segment (start 144.272 97.79) (end 146.685 97.79) (width 0.5) (layer B.Cu) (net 2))
 (segment (start 142.24 99.822) (end 144.272 97.79) (width 0.5) (layer B.Cu) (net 2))
 (segment (start 177.8 86.36) (end 177.8 98.298) (width 0.25) (layer B.Cu) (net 2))
 (segment (start 179.959 102.91064) (end 182.1688 105.12044) (width 0.25) (layer B.Cu) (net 2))
 (segment (start 179.959 100.457) (end 179.959 102.91064) (width 0.25) (layer B.Cu) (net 2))
 (segment (start 177.8 98.298) (end 179.959 100.457) (width 0.25) (layer B.Cu) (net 2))
 (segment (start 177.927 86.487) (end 177.8 86.36) (width 0.25) (layer B.Cu) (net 2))
 (segment (start 163.957 99.187) (end 163.957 98.425) (width 0.25) (layer B.Cu) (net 2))
 (segment (start 163.957 98.425) (end 164.592 97.79) (width 0.25) (layer B.Cu) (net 2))
 (segment (start 146.685 97.79) (end 164.592 97.79) (width 0.5) (layer B.Cu) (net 2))
 (segment (start 164.592 97.79) (end 166.37 97.79) (width 0.5) (layer B.Cu) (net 2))
 (segment (start 166.37 97.79) (end 177.8 86.36) (width 0.5) (layer B.Cu) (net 2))
 (segment (start 199.4662 100.61956) (end 199.4662 97.59696) (width 0.25) (layer B.Cu) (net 2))
 (segment (start 199.4662 97.59696) (end 198.46544 96.5962) (width 0.25) (layer B.Cu) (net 2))
 (segment (start 182.1688 105.12044) (end 182.1688 103.5812) (width 0.25) (layer B.Cu) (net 2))
 (segment (start 182.1688 103.5812) (end 183.007 102.743) (width 0.25) (layer B.Cu) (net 2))
 (segment (start 183.007 102.743) (end 197.34276 102.743) (width 0.25) (layer B.Cu) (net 2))
 (segment (start 197.34276 102.743) (end 199.4662 100.61956) (width 0.25) (layer B.Cu) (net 2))
 (segment (start 163.957 99.441) (end 163.957 99.187) (width 0.25) (layer B.Cu) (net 2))
 (segment (start 163.957 102.743) (end 162.56 104.14) (width 0.25) (layer B.Cu) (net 2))
 (segment (start 163.957 99.441) (end 163.957 102.743) (width 0.25) (layer B.Cu) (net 2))
 (segment (start 167.64 104.14) (end 170.18 104.14) (width 0.25) (layer F.Cu) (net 12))
 (segment (start 170.18 104.14) (end 172.72 101.6) (width 0.25) (layer F.Cu) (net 12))
 (segment (start 116.205 92.71) (end 139.954 92.71) (width 2) (layer F.Cu) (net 1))
 (segment (start 142.494 90.17) (end 146.685 90.17) (width 2) (layer F.Cu) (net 1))
 (segment (start 139.954 92.71) (end 142.494 90.17) (width 2) (layer F.Cu) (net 1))
 (segment (start 116.205 92.71) (end 139.954 92.71) (width 2) (layer B.Cu) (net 1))
 (segment (start 142.621 90.043) (end 146.558 90.043) (width 2) (layer B.Cu) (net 1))
 (segment (start 139.954 92.71) (end 142.621 90.043) (width 2) (layer B.Cu) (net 1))
 (segment (start 146.558 90.043) (end 146.685 90.17) (width 2) (layer B.Cu) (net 1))
 (segment (start 146.685 90.17) (end 166.37 90.17) (width 0.5) (layer F.Cu) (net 1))
 (segment (start 166.37 90.17) (end 177.8 101.6) (width 0.5) (layer F.Cu) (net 1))
 (segment (start 146.685 92.71) (end 147.32 92.71) (width 0.25) (layer B.Cu) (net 3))
 (segment (start 147.32 92.71) (end 148.463 91.567) (width 0.25) (layer B.Cu) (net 3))
 (segment (start 148.463 87.503) (end 147.32 86.36) (width 0.25) (layer B.Cu) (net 3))
 (segment (start 148.463 91.567) (end 148.463 87.503) (width 0.25) (layer B.Cu) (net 3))
 (segment (start 144.78 101.6) (end 145.288 101.6) (width 0.25) (layer F.Cu) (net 4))
 (segment (start 145.288 101.6) (end 148.463 98.425) (width 0.25) (layer F.Cu) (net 4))
 (segment (start 148.463 97.028) (end 146.685 95.25) (width 0.25) (layer F.Cu) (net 4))
 (segment (start 148.463 98.425) (end 148.463 97.028) (width 0.25) (layer F.Cu) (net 4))
 (segment (start 144.78 101.6) (end 144.78 100.965) (width 0.25) (layer F.Cu) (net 4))
 (segment (start 193.96456 90.0938) (end 178.9938 90.0938) (width 0.25) (layer F.Cu) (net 5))
 (segment (start 178.9938 90.0938) (end 175.26 86.36) (width 0.25) (layer F.Cu) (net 5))
 (segment (start 192.9638 105.12044) (end 192.9638 103.3018) (width 0.25) (layer F.Cu) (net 6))
 (segment (start 177.165 90.805) (end 172.72 86.36) (width 0.25) (layer F.Cu) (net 6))
 (segment (start 189.611 90.805) (end 177.165 90.805) (width 0.25) (layer F.Cu) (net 6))
 (segment (start 190.881 92.075) (end 189.611 90.805) (width 0.25) (layer F.Cu) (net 6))
 (segment (start 190.881 101.219) (end 190.881 92.075) (width 0.25) (layer F.Cu) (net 6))
 (segment (start 192.9638 103.3018) (end 190.881 101.219) (width 0.25) (layer F.Cu) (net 6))
 (segment (start 188.6712 100.61956) (end 188.6712 92.6592) (width 0.25) (layer F.Cu) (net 7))
 (segment (start 175.387 91.567) (end 170.18 86.36) (width 0.25) (layer F.Cu) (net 7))
 (segment (start 187.579 91.567) (end 175.387 91.567) (width 0.25) (layer F.Cu) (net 7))
 (segment (start 188.6712 92.6592) (end 187.579 91.567) (width 0.25) (layer F.Cu) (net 7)))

